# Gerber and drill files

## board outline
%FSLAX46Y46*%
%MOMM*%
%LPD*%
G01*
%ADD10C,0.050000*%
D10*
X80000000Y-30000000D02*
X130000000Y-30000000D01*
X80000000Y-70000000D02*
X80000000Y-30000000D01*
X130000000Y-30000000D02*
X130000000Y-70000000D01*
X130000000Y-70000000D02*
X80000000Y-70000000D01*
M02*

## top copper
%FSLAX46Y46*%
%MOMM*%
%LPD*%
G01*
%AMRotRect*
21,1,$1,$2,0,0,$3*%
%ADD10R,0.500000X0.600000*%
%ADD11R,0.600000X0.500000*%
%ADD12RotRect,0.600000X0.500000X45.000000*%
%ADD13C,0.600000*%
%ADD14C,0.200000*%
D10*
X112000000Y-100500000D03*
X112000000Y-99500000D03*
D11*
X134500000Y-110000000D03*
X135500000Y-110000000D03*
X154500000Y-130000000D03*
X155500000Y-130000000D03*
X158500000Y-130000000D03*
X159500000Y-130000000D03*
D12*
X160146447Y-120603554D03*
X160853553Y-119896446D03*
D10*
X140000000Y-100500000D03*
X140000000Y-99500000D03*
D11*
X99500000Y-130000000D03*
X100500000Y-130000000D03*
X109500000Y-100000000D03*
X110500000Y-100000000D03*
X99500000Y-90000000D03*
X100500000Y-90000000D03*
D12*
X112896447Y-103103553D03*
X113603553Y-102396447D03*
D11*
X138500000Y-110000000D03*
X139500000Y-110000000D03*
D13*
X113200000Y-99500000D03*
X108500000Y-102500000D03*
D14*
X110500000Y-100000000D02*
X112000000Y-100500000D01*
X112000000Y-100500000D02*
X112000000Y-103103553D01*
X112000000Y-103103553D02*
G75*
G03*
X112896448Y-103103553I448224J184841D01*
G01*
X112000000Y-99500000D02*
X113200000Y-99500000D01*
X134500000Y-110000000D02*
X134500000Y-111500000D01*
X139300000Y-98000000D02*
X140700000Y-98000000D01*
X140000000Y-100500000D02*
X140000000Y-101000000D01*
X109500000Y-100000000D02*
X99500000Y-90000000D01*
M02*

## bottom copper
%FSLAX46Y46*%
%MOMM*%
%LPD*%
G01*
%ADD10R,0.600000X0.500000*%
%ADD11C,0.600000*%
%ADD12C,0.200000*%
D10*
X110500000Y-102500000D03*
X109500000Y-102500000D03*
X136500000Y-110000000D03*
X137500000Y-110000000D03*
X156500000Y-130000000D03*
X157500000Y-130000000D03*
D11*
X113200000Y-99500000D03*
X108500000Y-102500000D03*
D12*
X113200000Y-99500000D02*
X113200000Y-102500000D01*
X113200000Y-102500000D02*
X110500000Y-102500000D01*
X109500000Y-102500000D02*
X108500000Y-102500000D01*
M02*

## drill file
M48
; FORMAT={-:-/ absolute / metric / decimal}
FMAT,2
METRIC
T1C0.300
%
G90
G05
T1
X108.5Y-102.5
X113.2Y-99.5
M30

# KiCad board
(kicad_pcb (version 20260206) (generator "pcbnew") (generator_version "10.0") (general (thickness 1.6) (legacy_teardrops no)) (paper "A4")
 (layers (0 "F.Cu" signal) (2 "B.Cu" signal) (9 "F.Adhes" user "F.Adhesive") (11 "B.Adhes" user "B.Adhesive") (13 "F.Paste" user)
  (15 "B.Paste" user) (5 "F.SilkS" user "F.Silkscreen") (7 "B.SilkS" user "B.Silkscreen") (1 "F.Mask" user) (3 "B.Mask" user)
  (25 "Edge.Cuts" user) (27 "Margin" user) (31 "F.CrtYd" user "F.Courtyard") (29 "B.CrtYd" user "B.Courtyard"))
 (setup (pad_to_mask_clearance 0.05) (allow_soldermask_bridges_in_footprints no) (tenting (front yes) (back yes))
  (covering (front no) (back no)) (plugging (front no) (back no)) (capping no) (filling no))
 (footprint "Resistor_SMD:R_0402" (layer "F.Cu") (at 112 100 90)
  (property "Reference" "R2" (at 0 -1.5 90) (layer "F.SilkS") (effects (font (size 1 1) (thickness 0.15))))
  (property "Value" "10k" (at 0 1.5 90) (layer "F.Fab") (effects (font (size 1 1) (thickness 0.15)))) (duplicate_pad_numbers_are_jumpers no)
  (pad "1" smd rect (at -0.5 0 90) (size 0.6 0.5) (layers "F.Cu" "F.Mask" "F.Paste") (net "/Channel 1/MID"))
  (pad "2" smd rect (at 0.5 0 90) (size 0.6 0.5) (layers "F.Cu" "F.Mask" "F.Paste") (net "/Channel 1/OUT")))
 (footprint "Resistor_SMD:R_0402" (layer "F.Cu") (at 135 110)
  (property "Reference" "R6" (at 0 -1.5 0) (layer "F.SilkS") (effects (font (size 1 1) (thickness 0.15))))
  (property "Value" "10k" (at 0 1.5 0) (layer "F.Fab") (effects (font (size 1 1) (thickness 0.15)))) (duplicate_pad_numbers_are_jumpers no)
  (pad "1" smd rect (at -0.5 0) (size 0.6 0.5) (layers "F.Cu" "F.Mask" "F.Paste") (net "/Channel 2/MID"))
  (pad "2" smd rect (at 0.5 0) (size 0.6 0.5) (layers "F.Cu" "F.Mask" "F.Paste") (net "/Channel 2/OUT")))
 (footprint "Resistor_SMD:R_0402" (layer "F.Cu") (at 155 130)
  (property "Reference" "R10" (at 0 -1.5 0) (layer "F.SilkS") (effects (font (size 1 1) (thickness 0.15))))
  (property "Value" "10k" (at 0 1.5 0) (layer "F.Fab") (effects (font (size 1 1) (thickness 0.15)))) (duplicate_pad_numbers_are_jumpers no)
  (pad "1" smd rect (at -0.5 0) (size 0.6 0.5) (layers "F.Cu" "F.Mask" "F.Paste") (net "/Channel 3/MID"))
  (pad "2" smd rect (at 0.5 0) (size 0.6 0.5) (layers "F.Cu" "F.Mask" "F.Paste") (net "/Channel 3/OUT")))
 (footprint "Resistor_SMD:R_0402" (layer "F.Cu") (at 159 130)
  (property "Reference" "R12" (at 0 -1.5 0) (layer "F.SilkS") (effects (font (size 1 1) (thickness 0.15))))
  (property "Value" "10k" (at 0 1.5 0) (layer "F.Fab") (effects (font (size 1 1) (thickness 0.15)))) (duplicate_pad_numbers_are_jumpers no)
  (pad "1" smd rect (at -0.5 0) (size 0.6 0.5) (layers "F.Cu" "F.Mask" "F.Paste") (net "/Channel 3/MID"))
  (pad "2" smd rect (at 0.5 0) (size 0.6 0.5) (layers "F.Cu" "F.Mask" "F.Paste") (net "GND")))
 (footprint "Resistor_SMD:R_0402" (layer "F.Cu") (at 160.5 120.25 45)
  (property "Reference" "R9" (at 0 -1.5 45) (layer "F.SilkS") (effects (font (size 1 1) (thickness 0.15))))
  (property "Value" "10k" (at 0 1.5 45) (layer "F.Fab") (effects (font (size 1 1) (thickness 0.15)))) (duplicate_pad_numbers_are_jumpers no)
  (pad "1" smd rect (at -0.5 0.000001 45) (size 0.6 0.5) (layers "F.Cu" "F.Mask" "F.Paste") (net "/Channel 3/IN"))
  (pad "2" smd rect (at 0.5 -0.000001 45) (size 0.6 0.5) (layers "F.Cu" "F.Mask" "F.Paste") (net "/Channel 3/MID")))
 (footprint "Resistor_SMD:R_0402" (layer "F.Cu") (at 140 100 90)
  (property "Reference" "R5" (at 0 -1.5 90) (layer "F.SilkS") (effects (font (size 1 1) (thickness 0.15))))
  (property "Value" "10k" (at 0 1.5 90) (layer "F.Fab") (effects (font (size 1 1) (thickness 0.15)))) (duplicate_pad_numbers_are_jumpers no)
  (pad "1" smd rect (at -0.5 0 90) (size 0.6 0.5) (layers "F.Cu" "F.Mask" "F.Paste") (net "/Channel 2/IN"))
  (pad "2" smd rect (at 0.5 0 90) (size 0.6 0.5) (layers "F.Cu" "F.Mask" "F.Paste") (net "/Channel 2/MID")))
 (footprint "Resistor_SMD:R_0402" (layer "F.Cu") (at 100 130)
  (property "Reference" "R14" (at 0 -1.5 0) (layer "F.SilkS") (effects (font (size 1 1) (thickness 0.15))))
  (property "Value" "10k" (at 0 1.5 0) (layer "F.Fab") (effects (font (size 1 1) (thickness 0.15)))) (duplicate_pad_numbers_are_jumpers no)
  (pad "1" smd rect (at -0.5 0) (size 0.6 0.5) (layers "F.Cu" "F.Mask" "F.Paste") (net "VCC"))
  (pad "2" smd rect (at 0.5 0) (size 0.6 0.5) (layers "F.Cu" "F.Mask" "F.Paste") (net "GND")))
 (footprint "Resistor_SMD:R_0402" (layer "F.Cu") (at 110 100)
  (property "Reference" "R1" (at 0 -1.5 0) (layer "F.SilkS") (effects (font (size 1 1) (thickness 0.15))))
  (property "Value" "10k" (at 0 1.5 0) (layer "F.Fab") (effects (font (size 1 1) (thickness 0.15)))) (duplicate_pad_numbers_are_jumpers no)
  (pad "1" smd rect (at -0.5 0) (size 0.6 0.5) (layers "F.Cu" "F.Mask" "F.Paste") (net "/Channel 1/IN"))
  (pad "2" smd rect (at 0.5 0) (size 0.6 0.5) (layers "F.Cu" "F.Mask" "F.Paste") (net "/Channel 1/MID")))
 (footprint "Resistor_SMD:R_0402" (layer "F.Cu") (at 100 90)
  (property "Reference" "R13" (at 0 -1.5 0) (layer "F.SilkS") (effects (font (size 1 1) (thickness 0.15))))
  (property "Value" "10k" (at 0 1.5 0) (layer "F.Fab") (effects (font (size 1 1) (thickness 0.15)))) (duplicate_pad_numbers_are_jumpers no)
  (pad "1" smd rect (at -0.5 0) (size 0.6 0.5) (layers "F.Cu" "F.Mask" "F.Paste") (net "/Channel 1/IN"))
  (pad "2" smd rect (at 0.5 0) (size 0.6 0.5) (layers "F.Cu" "F.Mask" "F.Paste") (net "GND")))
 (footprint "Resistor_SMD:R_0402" (layer "F.Cu") (at 113.25 102.75 45)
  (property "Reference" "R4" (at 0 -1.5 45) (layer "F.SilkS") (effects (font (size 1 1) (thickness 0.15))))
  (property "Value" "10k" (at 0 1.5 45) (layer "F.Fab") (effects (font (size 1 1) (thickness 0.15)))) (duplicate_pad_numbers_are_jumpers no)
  (pad "1" smd rect (at -0.499999 0 45) (size 0.6 0.5) (layers "F.Cu" "F.Mask" "F.Paste") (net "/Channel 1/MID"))
  (pad "2" smd rect (at 0.499999 0 45) (size 0.6 0.5) (layers "F.Cu" "F.Mask" "F.Paste") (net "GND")))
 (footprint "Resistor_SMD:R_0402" (layer "F.Cu") (at 139 110)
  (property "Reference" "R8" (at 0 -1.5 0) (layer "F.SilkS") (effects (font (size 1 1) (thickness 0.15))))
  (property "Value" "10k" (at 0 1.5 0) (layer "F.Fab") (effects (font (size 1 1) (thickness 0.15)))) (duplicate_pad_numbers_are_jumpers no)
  (pad "1" smd rect (at -0.5 0) (size 0.6 0.5) (layers "F.Cu" "F.Mask" "F.Paste") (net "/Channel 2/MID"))
  (pad "2" smd rect (at 0.5 0) (size 0.6 0.5) (layers "F.Cu" "F.Mask" "F.Paste") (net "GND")))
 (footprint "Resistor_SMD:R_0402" (layer "B.Cu") (at 110 102.5 180)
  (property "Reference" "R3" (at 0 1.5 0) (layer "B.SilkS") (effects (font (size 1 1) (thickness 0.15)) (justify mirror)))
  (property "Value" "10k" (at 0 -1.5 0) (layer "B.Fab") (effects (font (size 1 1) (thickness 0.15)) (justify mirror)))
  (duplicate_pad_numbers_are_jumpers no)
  (pad "1" smd rect (at -0.5 0 180) (size 0.6 0.5) (layers "B.Cu" "B.Mask" "B.Paste") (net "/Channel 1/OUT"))
  (pad "2" smd rect (at 0.5 0 180) (size 0.6 0.5) (layers "B.Cu" "B.Mask" "B.Paste") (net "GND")))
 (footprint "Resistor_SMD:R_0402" (layer "B.Cu") (at 137 110)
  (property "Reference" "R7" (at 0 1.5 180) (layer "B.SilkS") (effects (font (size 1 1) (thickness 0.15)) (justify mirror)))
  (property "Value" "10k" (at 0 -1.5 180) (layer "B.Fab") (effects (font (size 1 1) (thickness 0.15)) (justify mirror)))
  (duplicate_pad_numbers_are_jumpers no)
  (pad "1" smd rect (at -0.5 0) (size 0.6 0.5) (layers "B.Cu" "B.Mask" "B.Paste") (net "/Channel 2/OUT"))
  (pad "2" smd rect (at 0.5 0) (size 0.6 0.5) (layers "B.Cu" "B.Mask" "B.Paste") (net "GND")))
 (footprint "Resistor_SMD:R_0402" (layer "B.Cu") (at 157 130)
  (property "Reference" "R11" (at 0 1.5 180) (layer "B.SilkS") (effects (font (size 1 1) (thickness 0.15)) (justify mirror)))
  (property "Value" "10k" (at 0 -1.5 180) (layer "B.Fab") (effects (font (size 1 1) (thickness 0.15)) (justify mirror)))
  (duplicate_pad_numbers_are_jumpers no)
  (pad "1" smd rect (at -0.5 0) (size 0.6 0.5) (layers "B.Cu" "B.Mask" "B.Paste") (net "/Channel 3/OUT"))
  (pad "2" smd rect (at 0.5 0) (size 0.6 0.5) (layers "B.Cu" "B.Mask" "B.Paste") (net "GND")))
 (gr_line (start 80 30) (end 130 30) (stroke (width 0.05) (type default)) (layer "Edge.Cuts"))
 (gr_line (start 80 70) (end 80 30) (stroke (width 0.05) (type default)) (layer "Edge.Cuts"))
 (gr_line (start 130 30) (end 130 70) (stroke (width 0.05) (type default)) (layer "Edge.Cuts"))
 (gr_line (start 130 70) (end 80 70) (stroke (width 0.05) (type default)) (layer "Edge.Cuts"))
 (segment (start 110.5 100) (end 112 100.5) (width 0.2) (locked yes) (layer "F.Cu") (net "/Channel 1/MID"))
 (segment (start 112 100.5) (end 112 103.103553) (width 0.2) (layer "F.Cu") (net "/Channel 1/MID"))
 (arc (start 112 103.103553) (mid 112.448223 103.403553) (end 112.896447 103.103553) (width 0.2) (layer "F.Cu") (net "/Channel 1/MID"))
 (segment (start 112 99.5) (end 113.2 99.5) (width 0.2) (layer "F.Cu") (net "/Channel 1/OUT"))
 (via (at 113.2 99.5) (size 0.6) (drill 0.3) (layers "F.Cu" "B.Cu") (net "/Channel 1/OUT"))
 (segment (start 113.2 99.5) (end 113.2 102.5) (width 0.2) (layer "B.Cu") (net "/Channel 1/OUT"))
 (segment (start 113.2 102.5) (end 110.5 102.5) (width 0.2) (layer "B.Cu") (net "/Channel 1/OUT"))
 (segment (start 134.5 110) (end 134.5 111.5) (width 0.2) (layer "F.Cu") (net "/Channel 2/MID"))
 (segment (start 139.3 98) (end 140.7 98) (width 0.2) (layer "F.Cu") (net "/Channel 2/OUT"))
 (via (at 108.5 102.5) (size 0.6) (drill 0.3) (layers "F.Cu" "B.Cu") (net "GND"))
 (segment (start 109.5 102.5) (end 108.5 102.5) (width 0.2) (layer "B.Cu") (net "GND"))
 (segment (start 140 100.5) (end 140 101) (width 0.2) (layer "F.Cu") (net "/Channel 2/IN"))
 (segment (start 109.5 100) (end 99.5 90) (width 0.2) (layer "F.Cu") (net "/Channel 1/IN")))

